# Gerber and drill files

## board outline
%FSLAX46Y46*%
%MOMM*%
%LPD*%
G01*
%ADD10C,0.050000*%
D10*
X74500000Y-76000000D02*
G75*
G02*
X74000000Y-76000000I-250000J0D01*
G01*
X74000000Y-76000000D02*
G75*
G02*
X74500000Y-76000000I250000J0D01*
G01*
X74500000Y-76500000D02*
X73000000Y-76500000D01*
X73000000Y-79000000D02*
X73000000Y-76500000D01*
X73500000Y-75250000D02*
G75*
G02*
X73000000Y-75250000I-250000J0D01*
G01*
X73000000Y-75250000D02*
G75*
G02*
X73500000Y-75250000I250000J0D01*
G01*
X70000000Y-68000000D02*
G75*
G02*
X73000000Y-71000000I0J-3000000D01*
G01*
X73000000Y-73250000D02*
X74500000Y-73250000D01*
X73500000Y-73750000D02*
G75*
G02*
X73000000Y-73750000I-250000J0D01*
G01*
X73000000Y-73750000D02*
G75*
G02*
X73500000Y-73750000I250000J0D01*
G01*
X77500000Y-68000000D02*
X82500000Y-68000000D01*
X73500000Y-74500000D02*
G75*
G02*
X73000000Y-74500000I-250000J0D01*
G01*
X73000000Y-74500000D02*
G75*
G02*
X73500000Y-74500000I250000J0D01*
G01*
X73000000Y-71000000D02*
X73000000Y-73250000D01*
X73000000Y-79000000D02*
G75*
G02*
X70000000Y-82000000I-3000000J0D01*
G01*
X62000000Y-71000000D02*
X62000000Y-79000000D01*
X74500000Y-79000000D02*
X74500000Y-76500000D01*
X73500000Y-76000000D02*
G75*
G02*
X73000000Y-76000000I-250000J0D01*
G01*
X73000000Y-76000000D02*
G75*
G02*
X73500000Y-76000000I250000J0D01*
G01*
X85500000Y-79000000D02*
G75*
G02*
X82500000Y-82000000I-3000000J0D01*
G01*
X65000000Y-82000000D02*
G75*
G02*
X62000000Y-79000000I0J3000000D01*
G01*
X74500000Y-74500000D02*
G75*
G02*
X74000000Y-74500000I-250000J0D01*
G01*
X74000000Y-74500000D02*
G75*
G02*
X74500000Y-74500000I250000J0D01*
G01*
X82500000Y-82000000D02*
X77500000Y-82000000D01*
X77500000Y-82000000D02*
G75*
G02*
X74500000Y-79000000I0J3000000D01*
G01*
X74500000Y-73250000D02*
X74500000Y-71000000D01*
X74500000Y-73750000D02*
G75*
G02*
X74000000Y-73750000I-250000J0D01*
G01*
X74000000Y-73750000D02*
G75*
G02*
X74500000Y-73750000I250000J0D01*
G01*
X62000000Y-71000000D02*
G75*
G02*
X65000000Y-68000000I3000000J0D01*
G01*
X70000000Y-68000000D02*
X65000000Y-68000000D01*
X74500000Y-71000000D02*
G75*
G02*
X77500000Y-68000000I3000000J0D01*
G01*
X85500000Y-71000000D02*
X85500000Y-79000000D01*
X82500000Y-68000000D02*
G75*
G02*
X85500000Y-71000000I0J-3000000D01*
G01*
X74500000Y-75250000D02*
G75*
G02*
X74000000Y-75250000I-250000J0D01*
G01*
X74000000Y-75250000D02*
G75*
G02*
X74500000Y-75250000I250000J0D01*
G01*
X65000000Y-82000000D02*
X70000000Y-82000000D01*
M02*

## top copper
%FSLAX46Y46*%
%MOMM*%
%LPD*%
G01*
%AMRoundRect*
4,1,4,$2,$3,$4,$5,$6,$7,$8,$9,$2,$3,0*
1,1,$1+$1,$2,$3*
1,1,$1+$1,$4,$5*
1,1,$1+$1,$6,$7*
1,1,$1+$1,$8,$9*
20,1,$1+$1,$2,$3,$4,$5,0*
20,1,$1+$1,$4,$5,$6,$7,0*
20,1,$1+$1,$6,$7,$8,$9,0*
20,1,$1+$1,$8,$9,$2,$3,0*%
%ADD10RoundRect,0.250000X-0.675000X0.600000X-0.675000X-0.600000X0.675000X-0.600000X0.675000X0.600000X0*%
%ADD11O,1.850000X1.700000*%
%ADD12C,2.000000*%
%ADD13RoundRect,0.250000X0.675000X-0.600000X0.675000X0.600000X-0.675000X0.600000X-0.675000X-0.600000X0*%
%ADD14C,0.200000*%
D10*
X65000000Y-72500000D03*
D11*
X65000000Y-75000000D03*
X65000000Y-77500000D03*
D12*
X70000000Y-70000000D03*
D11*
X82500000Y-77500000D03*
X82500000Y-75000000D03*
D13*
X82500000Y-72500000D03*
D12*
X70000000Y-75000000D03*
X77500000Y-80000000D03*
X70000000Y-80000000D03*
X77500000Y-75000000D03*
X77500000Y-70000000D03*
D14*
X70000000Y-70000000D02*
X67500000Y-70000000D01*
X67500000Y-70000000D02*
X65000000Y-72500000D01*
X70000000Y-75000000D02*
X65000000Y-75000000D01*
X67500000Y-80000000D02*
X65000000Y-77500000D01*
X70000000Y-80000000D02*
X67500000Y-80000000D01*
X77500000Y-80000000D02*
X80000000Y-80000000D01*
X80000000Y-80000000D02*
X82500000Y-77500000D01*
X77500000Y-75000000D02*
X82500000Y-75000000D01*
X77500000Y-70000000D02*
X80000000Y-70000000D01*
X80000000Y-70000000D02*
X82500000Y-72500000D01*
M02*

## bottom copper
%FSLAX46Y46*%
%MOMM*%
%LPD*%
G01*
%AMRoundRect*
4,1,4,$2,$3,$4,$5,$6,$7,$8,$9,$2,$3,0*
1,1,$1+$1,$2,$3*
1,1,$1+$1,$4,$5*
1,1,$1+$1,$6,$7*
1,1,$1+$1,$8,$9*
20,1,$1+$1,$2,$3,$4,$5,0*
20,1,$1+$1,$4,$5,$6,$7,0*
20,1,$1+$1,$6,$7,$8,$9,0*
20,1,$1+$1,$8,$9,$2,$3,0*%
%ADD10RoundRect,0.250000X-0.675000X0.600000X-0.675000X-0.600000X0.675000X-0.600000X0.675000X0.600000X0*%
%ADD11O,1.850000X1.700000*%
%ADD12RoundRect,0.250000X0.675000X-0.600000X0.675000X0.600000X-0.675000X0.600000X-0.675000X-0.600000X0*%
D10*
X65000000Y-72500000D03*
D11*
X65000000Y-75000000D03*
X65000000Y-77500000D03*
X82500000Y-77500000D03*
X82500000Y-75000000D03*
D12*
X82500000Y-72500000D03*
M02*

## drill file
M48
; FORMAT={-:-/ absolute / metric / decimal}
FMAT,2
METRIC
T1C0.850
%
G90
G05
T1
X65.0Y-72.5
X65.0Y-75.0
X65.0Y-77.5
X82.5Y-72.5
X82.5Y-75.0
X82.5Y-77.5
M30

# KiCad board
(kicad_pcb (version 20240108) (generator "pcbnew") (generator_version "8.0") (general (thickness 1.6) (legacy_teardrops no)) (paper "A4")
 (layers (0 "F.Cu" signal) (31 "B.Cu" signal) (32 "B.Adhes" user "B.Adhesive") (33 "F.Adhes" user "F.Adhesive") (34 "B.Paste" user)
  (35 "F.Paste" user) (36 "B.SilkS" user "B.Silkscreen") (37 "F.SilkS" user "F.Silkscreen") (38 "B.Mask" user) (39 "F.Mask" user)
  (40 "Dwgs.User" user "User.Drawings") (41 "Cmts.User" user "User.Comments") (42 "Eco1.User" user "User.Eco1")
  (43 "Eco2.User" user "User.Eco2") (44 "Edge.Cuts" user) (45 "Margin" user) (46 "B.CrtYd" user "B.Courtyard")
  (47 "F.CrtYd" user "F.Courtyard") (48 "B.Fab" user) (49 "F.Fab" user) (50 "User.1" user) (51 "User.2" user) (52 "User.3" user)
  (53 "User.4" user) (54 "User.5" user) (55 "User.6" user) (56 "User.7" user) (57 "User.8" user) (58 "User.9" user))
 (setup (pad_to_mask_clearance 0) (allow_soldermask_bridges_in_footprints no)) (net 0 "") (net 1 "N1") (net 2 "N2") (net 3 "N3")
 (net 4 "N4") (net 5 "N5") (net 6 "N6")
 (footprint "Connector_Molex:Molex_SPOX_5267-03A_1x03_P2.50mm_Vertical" (layer "F.Cu") (at 65 72.5 -90)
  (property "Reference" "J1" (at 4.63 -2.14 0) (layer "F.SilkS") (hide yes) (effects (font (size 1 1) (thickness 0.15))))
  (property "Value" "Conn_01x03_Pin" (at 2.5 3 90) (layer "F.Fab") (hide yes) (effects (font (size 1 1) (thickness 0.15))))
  (pad "1" thru_hole roundrect (at 0 0 270) (size 1.7 1.85) (drill 0.85) (layers "*.Cu" "*.Mask") (remove_unused_layers no)
   (roundrect_rratio 0.147059) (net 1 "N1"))
  (pad "2" thru_hole oval (at 2.5 0 270) (size 1.7 1.85) (drill 0.85) (layers "*.Cu" "*.Mask") (remove_unused_layers no) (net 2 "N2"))
  (pad "3" thru_hole oval (at 5 0 270) (size 1.7 1.85) (drill 0.85) (layers "*.Cu" "*.Mask") (remove_unused_layers no) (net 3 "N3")))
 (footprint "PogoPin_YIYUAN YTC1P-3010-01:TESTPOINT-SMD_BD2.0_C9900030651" (layer "F.Cu") (at 70 70)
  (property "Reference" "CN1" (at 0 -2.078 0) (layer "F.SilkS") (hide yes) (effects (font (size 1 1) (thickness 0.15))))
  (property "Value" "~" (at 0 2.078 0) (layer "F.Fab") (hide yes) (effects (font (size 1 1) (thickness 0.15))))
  (pad "1" smd circle (at 0 0) (size 2 2) (layers "F.Cu" "F.Paste" "F.Mask") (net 1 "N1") (thermal_bridge_angle 90)))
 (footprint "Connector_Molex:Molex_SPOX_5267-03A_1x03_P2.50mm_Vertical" (layer "F.Cu") (at 82.5 77.5 90)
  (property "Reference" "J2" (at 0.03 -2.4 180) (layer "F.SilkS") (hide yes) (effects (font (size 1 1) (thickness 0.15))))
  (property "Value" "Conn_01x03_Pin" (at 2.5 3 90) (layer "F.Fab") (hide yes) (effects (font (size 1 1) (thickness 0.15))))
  (pad "1" thru_hole oval (at 0 0 90) (size 1.7 1.85) (drill 0.85) (layers "*.Cu" "*.Mask") (remove_unused_layers no) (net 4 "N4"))
  (pad "2" thru_hole oval (at 2.5 0 90) (size 1.7 1.85) (drill 0.85) (layers "*.Cu" "*.Mask") (remove_unused_layers no) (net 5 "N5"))
  (pad "3" thru_hole roundrect (at 5 0 90) (size 1.7 1.85) (drill 0.85) (layers "*.Cu" "*.Mask") (remove_unused_layers no)
   (roundrect_rratio 0.1470588235) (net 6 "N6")))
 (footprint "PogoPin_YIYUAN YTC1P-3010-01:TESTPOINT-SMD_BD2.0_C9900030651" (layer "F.Cu") (at 70 75)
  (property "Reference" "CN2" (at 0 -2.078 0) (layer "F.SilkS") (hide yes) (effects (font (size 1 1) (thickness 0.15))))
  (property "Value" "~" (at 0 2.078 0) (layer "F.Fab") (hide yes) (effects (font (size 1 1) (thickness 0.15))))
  (pad "1" smd circle (at 0 0) (size 2 2) (layers "F.Cu" "F.Paste" "F.Mask") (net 2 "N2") (thermal_bridge_angle 90)))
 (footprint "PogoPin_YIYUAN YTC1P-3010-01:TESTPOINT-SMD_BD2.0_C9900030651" (layer "F.Cu") (at 77.5 80)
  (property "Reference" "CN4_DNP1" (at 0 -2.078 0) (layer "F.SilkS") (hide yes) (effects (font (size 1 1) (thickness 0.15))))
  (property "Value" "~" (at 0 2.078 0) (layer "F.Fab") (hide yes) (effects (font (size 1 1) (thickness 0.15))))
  (pad "1" smd circle (at 0 0) (size 2 2) (layers "F.Cu" "F.Mask") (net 4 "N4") (thermal_bridge_angle 90)))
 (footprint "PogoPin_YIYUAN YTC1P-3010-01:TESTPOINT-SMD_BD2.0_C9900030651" (layer "F.Cu") (at 70 80)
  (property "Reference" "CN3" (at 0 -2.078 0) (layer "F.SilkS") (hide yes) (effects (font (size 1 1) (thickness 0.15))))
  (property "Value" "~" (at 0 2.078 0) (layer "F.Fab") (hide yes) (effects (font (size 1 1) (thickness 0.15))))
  (pad "1" smd circle (at 0 0) (size 2 2) (layers "F.Cu" "F.Paste" "F.Mask") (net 3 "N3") (thermal_bridge_angle 90)))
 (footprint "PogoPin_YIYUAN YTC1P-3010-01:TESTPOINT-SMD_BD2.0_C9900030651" (layer "F.Cu") (at 77.5 75)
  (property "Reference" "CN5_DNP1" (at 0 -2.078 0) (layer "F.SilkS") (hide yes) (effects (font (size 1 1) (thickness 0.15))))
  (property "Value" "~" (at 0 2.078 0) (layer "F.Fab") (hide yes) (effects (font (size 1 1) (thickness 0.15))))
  (pad "1" smd circle (at 0 0) (size 2 2) (layers "F.Cu" "F.Mask") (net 5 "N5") (thermal_bridge_angle 90)))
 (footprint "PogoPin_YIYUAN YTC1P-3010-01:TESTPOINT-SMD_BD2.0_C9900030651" (layer "F.Cu") (at 77.5 70)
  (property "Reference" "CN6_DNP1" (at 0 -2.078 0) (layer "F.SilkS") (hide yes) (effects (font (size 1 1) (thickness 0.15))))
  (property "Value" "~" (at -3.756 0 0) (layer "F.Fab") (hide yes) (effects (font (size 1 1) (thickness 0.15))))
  (pad "1" smd circle (at 0 0) (size 2 2) (layers "F.Cu" "F.Mask") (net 6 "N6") (thermal_bridge_angle 90)))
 (gr_circle (center 74.25 76) (end 74.25 76.25) (stroke (width 0.05) (type default)) (fill none) (layer "Edge.Cuts"))
 (gr_line (start 74.5 76.5) (end 73 76.5) (stroke (width 0.05) (type default)) (layer "Edge.Cuts"))
 (gr_line (start 73 79) (end 73 76.5) (stroke (width 0.05) (type default)) (layer "Edge.Cuts"))
 (gr_circle (center 73.25 75.25) (end 73.25 75.5) (stroke (width 0.05) (type default)) (fill none) (layer "Edge.Cuts"))
 (gr_arc (start 70 68) (mid 72.12132 68.87868) (end 73 71) (stroke (width 0.05) (type default)) (layer "Edge.Cuts"))
 (gr_line (start 73 73.25) (end 74.5 73.25) (stroke (width 0.05) (type default)) (layer "Edge.Cuts"))
 (gr_circle (center 73.25 73.75) (end 73.25 74) (stroke (width 0.05) (type default)) (fill none) (layer "Edge.Cuts"))
 (gr_line (start 77.5 68) (end 82.5 68) (stroke (width 0.05) (type default)) (layer "Edge.Cuts"))
 (gr_circle (center 73.25 74.5) (end 73.25 74.75) (stroke (width 0.05) (type default)) (fill none) (layer "Edge.Cuts"))
 (gr_line (start 73 71) (end 73 73.25) (stroke (width 0.05) (type default)) (layer "Edge.Cuts"))
 (gr_arc (start 73 79) (mid 72.12132 81.12132) (end 70 82) (stroke (width 0.05) (type default)) (layer "Edge.Cuts"))
 (gr_line (start 62 71) (end 62 79) (stroke (width 0.05) (type default)) (layer "Edge.Cuts"))
 (gr_line (start 74.5 79) (end 74.5 76.5) (stroke (width 0.05) (type default)) (layer "Edge.Cuts"))
 (gr_circle (center 73.25 76) (end 73.25 76.25) (stroke (width 0.05) (type default)) (fill none) (layer "Edge.Cuts"))
 (gr_arc (start 85.5 79) (mid 84.62132 81.12132) (end 82.5 82) (stroke (width 0.05) (type default)) (layer "Edge.Cuts"))
 (gr_arc (start 65 82) (mid 62.87868 81.12132) (end 62 79) (stroke (width 0.05) (type default)) (layer "Edge.Cuts"))
 (gr_circle (center 74.25 74.5) (end 74.25 74.75) (stroke (width 0.05) (type default)) (fill none) (layer "Edge.Cuts"))
 (gr_line (start 82.5 82) (end 77.5 82) (stroke (width 0.05) (type default)) (layer "Edge.Cuts"))
 (gr_arc (start 77.5 82) (mid 75.37868 81.12132) (end 74.5 79) (stroke (width 0.05) (type default)) (layer "Edge.Cuts"))
 (gr_line (start 74.5 73.25) (end 74.5 71) (stroke (width 0.05) (type default)) (layer "Edge.Cuts"))
 (gr_circle (center 74.25 73.75) (end 74.25 74) (stroke (width 0.05) (type default)) (fill none) (layer "Edge.Cuts"))
 (gr_arc (start 62 71) (mid 62.87868 68.87868) (end 65 68) (stroke (width 0.05) (type default)) (layer "Edge.Cuts"))
 (gr_line (start 70 68) (end 65 68) (stroke (width 0.05) (type default)) (layer "Edge.Cuts"))
 (gr_arc (start 74.5 71) (mid 75.37868 68.87868) (end 77.5 68) (stroke (width 0.05) (type default)) (layer "Edge.Cuts"))
 (gr_line (start 85.5 71) (end 85.5 79) (stroke (width 0.05) (type default)) (layer "Edge.Cuts"))
 (gr_arc (start 82.5 68) (mid 84.62132 68.87868) (end 85.5 71) (stroke (width 0.05) (type default)) (layer "Edge.Cuts"))
 (gr_circle (center 74.25 75.25) (end 74.25 75.5) (stroke (width 0.05) (type default)) (fill none) (layer "Edge.Cuts"))
 (gr_line (start 65 82) (end 70 82) (stroke (width 0.05) (type default)) (layer "Edge.Cuts"))
 (segment (start 70 70) (end 67.5 70) (width 0.2) (layer "F.Cu") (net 1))
 (segment (start 67.5 70) (end 65 72.5) (width 0.2) (layer "F.Cu") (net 1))
 (segment (start 70 75) (end 65 75) (width 0.2) (layer "F.Cu") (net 2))
 (segment (start 67.5 80) (end 65 77.5) (width 0.2) (layer "F.Cu") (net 3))
 (segment (start 70 80) (end 67.5 80) (width 0.2) (layer "F.Cu") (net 3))
 (segment (start 77.5 80) (end 80 80) (width 0.2) (layer "F.Cu") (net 4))
 (segment (start 80 80) (end 82.5 77.5) (width 0.2) (layer "F.Cu") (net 4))
 (segment (start 77.5 75) (end 82.5 75) (width 0.2) (layer "F.Cu") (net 5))
 (segment (start 77.5 70) (end 80 70) (width 0.2) (layer "F.Cu") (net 6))
 (segment (start 80 70) (end 82.5 72.5) (width 0.2) (layer "F.Cu") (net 6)))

